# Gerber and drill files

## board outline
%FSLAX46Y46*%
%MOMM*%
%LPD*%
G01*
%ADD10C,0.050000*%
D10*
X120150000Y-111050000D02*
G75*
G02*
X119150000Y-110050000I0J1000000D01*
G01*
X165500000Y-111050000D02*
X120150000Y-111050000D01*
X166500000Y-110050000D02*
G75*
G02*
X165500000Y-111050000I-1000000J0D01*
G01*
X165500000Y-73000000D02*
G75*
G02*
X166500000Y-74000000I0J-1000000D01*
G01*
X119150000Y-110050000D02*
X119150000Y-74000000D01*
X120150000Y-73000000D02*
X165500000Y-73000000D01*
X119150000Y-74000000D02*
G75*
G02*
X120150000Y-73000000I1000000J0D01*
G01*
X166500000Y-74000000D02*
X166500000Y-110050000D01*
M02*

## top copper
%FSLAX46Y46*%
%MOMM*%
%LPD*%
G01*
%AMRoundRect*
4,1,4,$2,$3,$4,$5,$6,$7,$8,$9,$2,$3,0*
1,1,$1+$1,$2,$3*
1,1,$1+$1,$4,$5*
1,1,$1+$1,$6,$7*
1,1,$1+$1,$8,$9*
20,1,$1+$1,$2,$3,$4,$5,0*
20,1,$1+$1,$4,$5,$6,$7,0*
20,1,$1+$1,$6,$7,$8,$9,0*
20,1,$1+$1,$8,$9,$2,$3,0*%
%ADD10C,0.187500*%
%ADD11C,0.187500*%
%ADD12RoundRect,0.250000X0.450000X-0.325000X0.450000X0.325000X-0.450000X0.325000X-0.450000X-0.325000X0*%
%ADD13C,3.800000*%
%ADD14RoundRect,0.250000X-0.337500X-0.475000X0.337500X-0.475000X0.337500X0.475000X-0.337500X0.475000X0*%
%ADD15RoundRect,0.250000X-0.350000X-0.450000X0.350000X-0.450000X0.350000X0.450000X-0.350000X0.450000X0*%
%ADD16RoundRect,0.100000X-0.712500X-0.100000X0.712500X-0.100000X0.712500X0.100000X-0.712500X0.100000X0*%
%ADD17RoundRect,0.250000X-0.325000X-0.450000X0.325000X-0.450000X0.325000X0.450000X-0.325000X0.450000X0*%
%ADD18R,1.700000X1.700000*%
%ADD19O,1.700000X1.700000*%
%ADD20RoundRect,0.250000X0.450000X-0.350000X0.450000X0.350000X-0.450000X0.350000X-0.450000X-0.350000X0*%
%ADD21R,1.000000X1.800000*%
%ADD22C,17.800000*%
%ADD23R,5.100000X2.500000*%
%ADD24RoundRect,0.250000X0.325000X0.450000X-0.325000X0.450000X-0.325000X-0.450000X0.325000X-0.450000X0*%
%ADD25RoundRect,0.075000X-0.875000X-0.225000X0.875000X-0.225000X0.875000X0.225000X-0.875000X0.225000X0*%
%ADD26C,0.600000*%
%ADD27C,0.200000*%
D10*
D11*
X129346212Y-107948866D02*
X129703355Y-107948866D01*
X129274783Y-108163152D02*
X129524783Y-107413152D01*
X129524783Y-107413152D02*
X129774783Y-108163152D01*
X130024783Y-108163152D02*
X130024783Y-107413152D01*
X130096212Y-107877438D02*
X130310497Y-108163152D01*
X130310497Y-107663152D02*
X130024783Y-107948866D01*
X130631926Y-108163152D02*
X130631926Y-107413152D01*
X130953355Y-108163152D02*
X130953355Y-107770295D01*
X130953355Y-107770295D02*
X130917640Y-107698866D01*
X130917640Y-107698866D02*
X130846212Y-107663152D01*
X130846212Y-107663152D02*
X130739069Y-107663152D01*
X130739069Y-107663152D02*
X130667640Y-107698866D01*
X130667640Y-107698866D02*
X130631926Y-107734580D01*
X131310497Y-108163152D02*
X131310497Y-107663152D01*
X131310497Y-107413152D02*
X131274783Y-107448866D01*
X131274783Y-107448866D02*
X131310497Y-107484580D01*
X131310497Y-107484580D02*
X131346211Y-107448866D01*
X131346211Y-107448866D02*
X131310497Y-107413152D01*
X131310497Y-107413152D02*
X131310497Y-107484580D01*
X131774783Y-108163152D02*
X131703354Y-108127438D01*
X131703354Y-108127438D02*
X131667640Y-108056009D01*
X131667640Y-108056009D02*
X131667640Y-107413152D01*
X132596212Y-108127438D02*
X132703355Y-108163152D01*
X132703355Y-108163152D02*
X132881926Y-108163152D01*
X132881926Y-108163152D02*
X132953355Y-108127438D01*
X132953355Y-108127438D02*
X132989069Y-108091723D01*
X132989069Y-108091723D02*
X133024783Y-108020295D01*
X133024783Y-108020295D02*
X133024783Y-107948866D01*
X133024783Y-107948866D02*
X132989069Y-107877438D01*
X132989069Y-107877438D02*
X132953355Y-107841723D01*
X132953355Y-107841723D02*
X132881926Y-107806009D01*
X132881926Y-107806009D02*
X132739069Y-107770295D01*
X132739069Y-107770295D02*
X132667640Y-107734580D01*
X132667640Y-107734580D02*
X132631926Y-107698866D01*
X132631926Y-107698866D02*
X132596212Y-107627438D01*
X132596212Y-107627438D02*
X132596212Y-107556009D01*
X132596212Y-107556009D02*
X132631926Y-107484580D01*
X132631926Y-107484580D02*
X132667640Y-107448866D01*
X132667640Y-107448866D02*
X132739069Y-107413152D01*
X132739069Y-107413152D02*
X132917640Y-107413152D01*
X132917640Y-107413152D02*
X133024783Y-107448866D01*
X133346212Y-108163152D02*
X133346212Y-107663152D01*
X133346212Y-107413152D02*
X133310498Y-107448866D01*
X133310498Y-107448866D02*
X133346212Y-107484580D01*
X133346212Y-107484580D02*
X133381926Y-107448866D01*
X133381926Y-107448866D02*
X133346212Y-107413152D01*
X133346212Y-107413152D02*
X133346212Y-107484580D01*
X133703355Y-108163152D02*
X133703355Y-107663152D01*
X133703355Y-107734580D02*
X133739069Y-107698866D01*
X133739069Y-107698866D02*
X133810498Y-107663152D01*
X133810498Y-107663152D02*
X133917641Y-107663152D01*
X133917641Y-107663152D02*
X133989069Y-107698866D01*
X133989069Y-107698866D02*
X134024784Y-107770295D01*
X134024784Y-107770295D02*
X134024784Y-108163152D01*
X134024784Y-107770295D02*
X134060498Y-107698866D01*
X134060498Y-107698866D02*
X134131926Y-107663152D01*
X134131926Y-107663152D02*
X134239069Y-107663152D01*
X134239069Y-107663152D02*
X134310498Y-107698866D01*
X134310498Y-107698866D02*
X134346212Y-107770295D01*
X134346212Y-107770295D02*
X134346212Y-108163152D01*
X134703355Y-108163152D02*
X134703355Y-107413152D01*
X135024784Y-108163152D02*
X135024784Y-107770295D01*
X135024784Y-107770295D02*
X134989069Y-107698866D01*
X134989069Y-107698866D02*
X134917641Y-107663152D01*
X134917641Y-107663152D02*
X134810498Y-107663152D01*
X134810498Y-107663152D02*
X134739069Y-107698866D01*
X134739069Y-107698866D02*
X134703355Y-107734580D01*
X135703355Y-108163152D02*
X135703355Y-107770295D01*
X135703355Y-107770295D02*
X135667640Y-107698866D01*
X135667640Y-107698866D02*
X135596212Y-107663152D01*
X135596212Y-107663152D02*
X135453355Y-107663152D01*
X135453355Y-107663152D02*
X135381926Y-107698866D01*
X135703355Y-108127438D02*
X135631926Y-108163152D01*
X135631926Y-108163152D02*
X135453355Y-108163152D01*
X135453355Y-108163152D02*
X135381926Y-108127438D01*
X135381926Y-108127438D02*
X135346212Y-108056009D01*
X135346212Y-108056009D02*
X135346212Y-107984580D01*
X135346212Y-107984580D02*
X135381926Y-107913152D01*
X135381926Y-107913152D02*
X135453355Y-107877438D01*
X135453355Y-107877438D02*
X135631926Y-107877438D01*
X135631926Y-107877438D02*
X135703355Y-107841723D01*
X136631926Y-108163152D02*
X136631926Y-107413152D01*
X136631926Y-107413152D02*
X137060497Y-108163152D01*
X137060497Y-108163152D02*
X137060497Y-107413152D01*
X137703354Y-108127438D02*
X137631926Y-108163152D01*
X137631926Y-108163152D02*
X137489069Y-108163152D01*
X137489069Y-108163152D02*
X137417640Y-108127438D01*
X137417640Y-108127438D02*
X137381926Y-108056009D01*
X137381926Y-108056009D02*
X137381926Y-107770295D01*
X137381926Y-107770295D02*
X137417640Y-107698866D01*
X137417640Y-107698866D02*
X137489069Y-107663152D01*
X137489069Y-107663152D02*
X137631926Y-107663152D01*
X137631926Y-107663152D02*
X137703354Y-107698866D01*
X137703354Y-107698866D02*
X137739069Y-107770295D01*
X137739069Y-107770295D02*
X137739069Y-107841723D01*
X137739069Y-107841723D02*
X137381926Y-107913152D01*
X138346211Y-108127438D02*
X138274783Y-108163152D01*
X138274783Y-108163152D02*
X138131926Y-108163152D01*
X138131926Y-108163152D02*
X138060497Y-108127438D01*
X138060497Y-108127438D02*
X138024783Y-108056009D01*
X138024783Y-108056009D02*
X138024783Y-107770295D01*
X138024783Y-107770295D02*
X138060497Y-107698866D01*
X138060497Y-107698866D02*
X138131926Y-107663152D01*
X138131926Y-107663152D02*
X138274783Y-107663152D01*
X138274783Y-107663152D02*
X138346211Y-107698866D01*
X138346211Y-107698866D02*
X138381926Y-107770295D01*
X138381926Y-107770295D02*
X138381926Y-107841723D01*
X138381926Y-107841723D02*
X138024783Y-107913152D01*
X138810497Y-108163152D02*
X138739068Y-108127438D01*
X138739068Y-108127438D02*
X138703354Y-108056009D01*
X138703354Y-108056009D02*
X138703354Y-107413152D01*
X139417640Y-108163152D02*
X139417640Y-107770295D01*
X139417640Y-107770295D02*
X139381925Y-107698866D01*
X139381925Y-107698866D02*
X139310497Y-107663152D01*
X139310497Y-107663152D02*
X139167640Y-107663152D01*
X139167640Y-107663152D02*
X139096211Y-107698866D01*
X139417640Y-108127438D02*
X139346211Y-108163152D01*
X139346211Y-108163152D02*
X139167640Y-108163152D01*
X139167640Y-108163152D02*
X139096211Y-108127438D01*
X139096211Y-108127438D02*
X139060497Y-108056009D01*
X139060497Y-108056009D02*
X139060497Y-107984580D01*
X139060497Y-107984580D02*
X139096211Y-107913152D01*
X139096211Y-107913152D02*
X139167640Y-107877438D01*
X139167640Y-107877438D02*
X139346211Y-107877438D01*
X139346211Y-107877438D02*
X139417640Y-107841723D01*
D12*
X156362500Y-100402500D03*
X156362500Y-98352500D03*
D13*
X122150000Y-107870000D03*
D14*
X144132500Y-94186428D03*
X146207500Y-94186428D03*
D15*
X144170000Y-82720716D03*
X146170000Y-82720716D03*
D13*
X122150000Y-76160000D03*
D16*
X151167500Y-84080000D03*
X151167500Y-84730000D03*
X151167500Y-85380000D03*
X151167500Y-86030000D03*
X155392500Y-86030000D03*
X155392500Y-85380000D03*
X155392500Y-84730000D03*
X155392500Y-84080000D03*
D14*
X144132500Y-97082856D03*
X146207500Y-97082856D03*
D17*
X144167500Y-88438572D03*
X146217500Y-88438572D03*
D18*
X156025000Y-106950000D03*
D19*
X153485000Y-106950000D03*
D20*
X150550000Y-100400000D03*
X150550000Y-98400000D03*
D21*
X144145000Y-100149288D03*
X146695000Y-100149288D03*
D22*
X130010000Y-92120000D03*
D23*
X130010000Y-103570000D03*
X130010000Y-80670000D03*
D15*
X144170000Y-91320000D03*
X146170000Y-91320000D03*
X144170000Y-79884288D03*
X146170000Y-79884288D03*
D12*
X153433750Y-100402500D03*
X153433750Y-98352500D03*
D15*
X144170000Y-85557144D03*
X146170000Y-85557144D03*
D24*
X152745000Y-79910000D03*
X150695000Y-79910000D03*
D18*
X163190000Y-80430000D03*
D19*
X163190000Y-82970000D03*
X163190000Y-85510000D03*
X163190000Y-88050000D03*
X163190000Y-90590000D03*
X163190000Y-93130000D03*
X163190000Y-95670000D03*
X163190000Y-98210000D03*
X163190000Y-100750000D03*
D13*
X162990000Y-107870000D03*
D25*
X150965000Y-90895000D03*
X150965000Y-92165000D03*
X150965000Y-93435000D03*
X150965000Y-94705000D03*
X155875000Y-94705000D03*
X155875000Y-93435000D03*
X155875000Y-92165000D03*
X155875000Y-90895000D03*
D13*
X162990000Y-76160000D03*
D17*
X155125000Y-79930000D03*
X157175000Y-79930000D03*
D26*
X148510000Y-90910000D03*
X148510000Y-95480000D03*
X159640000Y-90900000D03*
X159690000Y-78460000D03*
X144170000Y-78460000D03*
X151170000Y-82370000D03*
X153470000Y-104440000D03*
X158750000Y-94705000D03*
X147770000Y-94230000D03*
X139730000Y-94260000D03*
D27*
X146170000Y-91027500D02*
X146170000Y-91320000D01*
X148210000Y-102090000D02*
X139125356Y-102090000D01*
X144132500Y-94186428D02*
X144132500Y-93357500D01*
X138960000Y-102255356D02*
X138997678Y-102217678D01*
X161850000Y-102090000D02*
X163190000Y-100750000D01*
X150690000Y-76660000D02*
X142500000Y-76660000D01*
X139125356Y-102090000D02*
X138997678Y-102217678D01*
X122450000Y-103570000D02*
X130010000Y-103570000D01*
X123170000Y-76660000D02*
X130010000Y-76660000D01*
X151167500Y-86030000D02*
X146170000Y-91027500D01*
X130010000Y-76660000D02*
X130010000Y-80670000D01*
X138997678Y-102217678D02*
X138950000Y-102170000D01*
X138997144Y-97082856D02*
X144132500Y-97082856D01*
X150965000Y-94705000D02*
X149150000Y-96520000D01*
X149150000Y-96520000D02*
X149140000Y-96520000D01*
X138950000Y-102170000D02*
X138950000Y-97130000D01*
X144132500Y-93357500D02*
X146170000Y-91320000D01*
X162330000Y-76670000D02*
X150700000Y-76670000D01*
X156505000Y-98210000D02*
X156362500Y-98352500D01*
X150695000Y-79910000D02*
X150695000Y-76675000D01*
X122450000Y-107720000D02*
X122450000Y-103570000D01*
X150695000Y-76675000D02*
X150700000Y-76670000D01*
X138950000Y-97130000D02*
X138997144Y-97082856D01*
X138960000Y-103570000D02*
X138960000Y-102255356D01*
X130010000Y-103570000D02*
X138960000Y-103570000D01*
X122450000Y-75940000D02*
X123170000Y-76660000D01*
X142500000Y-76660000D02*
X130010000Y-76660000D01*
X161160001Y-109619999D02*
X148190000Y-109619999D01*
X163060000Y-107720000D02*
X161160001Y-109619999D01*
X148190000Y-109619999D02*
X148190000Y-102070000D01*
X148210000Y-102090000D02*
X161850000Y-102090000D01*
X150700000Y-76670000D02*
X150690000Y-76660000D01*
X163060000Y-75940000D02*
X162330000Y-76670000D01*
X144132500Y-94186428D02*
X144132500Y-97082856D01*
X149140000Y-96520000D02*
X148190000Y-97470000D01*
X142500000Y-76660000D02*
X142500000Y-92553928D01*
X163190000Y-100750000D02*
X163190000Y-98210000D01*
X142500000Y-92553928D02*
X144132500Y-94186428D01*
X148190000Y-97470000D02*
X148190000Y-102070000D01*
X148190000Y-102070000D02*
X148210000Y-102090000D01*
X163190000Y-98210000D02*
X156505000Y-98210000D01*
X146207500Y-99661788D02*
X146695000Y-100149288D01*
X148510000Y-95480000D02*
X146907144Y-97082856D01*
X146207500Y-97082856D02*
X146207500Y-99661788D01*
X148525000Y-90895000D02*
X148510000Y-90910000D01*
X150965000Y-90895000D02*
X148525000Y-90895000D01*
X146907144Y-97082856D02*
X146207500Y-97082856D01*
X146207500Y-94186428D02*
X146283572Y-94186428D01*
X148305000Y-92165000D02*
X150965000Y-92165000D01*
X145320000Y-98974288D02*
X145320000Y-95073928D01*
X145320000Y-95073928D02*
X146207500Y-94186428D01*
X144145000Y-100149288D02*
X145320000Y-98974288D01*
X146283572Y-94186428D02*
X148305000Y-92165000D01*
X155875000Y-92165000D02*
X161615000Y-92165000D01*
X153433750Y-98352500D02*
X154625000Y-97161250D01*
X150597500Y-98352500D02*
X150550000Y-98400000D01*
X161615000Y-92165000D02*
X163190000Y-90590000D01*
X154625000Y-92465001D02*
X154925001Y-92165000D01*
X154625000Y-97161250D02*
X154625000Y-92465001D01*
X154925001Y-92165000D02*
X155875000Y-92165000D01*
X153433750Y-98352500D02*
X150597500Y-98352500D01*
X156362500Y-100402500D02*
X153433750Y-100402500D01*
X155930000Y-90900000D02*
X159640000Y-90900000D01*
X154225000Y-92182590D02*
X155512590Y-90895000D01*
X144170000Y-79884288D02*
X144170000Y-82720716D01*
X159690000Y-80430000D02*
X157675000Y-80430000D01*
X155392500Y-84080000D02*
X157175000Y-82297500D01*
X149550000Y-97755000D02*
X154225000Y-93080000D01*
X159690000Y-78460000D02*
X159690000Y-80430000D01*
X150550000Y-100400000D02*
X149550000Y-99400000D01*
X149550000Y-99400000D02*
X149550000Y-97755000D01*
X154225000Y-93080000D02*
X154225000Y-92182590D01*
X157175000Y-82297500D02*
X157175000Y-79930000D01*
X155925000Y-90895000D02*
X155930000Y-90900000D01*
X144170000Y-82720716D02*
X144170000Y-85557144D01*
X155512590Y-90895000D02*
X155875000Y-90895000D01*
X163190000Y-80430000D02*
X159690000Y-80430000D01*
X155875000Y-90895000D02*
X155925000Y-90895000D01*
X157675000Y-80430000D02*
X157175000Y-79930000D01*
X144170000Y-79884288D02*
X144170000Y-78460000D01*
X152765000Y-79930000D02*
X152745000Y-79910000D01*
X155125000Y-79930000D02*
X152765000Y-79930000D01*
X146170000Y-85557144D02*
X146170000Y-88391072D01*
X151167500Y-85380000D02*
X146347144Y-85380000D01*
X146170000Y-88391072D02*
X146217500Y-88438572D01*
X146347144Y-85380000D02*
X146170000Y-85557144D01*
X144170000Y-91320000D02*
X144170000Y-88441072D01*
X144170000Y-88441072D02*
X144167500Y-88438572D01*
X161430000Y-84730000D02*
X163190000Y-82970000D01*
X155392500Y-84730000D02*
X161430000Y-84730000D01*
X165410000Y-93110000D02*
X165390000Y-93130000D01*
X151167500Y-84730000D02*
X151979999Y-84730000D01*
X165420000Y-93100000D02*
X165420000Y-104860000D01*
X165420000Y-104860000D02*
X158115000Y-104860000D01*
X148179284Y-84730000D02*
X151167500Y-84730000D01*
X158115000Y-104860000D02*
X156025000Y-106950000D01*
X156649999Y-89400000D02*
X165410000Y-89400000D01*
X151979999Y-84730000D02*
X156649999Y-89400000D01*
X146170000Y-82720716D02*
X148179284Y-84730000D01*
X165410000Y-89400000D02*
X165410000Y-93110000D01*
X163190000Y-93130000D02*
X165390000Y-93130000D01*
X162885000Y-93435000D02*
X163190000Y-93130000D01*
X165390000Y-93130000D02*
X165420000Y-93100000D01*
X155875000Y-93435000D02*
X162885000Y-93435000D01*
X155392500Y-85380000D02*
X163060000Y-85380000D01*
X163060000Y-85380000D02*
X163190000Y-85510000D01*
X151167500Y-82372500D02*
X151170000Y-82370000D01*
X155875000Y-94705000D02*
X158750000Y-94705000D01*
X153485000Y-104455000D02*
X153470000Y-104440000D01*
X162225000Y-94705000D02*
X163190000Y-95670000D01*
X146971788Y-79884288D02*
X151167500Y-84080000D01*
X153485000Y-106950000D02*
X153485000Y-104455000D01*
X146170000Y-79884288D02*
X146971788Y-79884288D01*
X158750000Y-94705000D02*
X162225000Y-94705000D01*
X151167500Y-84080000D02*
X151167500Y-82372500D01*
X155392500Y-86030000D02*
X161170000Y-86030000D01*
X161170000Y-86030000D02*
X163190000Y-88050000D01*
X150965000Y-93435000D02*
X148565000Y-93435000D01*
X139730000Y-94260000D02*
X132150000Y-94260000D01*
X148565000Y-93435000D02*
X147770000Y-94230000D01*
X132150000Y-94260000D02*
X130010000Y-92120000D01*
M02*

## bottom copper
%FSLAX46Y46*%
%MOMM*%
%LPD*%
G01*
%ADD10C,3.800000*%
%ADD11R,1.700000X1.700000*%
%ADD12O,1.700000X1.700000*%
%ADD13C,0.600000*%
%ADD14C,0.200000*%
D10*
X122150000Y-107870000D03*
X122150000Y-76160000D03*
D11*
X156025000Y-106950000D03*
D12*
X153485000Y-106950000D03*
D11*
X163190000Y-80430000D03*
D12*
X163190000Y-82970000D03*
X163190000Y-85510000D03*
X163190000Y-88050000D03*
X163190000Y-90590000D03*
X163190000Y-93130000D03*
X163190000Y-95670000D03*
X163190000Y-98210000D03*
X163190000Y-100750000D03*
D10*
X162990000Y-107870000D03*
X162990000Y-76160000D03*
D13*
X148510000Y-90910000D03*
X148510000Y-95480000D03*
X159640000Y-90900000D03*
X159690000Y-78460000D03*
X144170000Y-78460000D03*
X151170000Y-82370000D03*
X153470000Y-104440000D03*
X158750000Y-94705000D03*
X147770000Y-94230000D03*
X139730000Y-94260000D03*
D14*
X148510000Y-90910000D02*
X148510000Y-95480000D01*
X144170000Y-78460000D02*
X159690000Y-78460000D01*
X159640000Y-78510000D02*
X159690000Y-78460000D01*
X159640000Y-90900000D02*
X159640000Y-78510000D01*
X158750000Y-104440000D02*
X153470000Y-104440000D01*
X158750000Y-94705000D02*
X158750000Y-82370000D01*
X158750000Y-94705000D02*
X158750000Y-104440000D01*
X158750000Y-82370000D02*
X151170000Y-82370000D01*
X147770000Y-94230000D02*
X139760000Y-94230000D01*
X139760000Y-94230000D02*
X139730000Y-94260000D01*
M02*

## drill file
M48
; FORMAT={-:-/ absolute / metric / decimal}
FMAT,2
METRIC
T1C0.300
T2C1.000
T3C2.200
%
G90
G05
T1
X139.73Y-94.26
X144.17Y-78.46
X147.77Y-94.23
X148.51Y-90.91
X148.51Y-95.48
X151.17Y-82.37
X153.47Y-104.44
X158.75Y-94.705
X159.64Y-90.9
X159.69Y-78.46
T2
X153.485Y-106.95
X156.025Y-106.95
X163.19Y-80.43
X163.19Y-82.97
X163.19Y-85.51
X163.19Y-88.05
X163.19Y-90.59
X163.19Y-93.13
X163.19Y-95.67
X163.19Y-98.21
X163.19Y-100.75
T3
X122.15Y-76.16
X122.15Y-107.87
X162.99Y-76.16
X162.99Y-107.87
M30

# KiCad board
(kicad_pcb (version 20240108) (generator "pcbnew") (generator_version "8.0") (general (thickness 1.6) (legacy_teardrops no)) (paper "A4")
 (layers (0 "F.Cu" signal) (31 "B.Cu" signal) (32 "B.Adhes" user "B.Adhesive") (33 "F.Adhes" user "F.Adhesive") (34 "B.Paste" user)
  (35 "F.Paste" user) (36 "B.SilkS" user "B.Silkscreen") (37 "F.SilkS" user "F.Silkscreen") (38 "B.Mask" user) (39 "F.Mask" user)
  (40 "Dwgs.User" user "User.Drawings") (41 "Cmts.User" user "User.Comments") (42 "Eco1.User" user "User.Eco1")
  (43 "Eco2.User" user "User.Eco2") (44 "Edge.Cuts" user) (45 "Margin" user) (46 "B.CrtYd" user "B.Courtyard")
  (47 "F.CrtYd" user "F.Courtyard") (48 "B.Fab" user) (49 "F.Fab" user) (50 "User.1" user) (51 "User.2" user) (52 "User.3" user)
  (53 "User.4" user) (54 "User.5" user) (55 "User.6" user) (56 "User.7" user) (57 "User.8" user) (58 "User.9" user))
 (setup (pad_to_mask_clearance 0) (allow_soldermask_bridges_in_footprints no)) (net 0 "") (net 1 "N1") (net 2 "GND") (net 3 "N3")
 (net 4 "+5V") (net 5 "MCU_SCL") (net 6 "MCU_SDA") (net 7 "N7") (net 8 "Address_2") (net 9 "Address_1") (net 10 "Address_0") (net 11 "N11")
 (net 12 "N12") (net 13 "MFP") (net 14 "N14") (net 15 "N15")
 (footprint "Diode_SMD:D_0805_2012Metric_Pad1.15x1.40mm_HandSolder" (layer "F.Cu") (at 156.3625 99.3775 90)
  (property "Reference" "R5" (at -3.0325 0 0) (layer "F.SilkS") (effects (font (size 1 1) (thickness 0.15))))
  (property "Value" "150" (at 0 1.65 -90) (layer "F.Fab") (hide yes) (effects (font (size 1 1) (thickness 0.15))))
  (pad "1" smd roundrect (at -1.025 0 90) (size 1.15 1.4) (layers "F.Cu" "F.Paste" "F.Mask") (roundrect_rratio 0.217391) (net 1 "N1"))
  (pad "2" smd roundrect (at 1.025 0 90) (size 1.15 1.4) (layers "F.Cu" "F.Paste" "F.Mask") (roundrect_rratio 0.217391) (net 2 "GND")))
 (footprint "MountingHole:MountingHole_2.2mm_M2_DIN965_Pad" (layer "F.Cu") (at 122.15 107.87)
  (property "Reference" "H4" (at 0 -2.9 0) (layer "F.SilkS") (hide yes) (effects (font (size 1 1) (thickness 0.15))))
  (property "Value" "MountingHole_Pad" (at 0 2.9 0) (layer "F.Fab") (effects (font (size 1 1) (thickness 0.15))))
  (pad "1" thru_hole circle (at 0 0) (size 3.8 3.8) (drill 2.2) (layers "*.Cu" "*.Mask") (remove_unused_layers no) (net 2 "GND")))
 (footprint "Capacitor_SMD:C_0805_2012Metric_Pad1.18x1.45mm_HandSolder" (layer "F.Cu") (at 145.17 94.186428)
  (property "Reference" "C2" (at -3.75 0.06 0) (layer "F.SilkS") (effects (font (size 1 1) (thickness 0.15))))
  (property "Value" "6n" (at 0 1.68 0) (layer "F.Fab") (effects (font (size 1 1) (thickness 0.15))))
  (pad "1" smd roundrect (at -1.0375 0) (size 1.175 1.45) (layers "F.Cu" "F.Paste" "F.Mask") (roundrect_rratio 0.212766) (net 2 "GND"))
  (pad "2" smd roundrect (at 1.0375 0) (size 1.175 1.45) (layers "F.Cu" "F.Paste" "F.Mask") (roundrect_rratio 0.212766) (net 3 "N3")))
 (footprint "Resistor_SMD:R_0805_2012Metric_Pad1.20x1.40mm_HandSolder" (layer "F.Cu") (at 145.17 82.720716)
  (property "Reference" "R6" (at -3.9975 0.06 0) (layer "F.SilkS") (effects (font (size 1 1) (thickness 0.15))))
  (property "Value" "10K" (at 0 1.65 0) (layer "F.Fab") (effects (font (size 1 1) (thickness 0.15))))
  (pad "1" smd roundrect (at -1 0) (size 1.2 1.4) (layers "F.Cu" "F.Paste" "F.Mask") (roundrect_rratio 0.208333) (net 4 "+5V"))
  (pad "2" smd roundrect (at 1 0) (size 1.2 1.4) (layers "F.Cu" "F.Paste" "F.Mask") (roundrect_rratio 0.208333) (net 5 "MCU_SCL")))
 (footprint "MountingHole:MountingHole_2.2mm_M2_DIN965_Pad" (layer "F.Cu") (at 122.15 76.16)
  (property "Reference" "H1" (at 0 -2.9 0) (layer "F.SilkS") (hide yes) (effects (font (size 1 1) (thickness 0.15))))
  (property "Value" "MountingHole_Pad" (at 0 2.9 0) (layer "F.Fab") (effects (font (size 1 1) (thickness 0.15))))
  (pad "1" thru_hole circle (at 0 0) (size 3.8 3.8) (drill 2.2) (layers "*.Cu" "*.Mask") (remove_unused_layers no) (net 2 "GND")))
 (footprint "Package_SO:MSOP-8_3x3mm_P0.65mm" (layer "F.Cu") (at 153.28 85.055)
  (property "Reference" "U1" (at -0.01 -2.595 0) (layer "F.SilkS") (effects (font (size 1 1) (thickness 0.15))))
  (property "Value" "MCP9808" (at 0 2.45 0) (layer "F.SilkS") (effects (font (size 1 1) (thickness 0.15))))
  (pad "1" smd roundrect (at -2.1125 -0.975) (size 1.625 0.4) (layers "F.Cu" "F.Paste" "F.Mask") (roundrect_rratio 0.25) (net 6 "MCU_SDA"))
  (pad "2" smd roundrect (at -2.1125 -0.325) (size 1.625 0.4) (layers "F.Cu" "F.Paste" "F.Mask") (roundrect_rratio 0.25) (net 5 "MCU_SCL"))
  (pad "3" smd roundrect (at -2.1125 0.325) (size 1.625 0.4) (layers "F.Cu" "F.Paste" "F.Mask") (roundrect_rratio 0.25) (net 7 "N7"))
  (pad "4" smd roundrect (at -2.1125 0.975) (size 1.625 0.4) (layers "F.Cu" "F.Paste" "F.Mask") (roundrect_rratio 0.25) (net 2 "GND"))
  (pad "5" smd roundrect (at 2.1125 0.975) (size 1.625 0.4) (layers "F.Cu" "F.Paste" "F.Mask") (roundrect_rratio 0.25) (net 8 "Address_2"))
  (pad "6" smd roundrect (at 2.1125 0.325) (size 1.625 0.4) (layers "F.Cu" "F.Paste" "F.Mask") (roundrect_rratio 0.25) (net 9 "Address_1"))
  (pad "7" smd roundrect (at 2.1125 -0.325) (size 1.625 0.4) (layers "F.Cu" "F.Paste" "F.Mask") (roundrect_rratio 0.25) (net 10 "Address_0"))
  (pad "8" smd roundrect (at 2.1125 -0.975) (size 1.625 0.4) (layers "F.Cu" "F.Paste" "F.Mask") (roundrect_rratio 0.25) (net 4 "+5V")))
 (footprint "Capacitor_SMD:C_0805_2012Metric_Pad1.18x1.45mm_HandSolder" (layer "F.Cu") (at 145.17 97.082856)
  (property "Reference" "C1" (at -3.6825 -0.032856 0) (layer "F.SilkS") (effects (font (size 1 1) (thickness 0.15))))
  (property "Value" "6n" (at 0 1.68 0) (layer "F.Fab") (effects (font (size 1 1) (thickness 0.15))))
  (pad "1" smd roundrect (at -1.0375 0) (size 1.175 1.45) (layers "F.Cu" "F.Paste" "F.Mask") (roundrect_rratio 0.212766) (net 2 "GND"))
  (pad "2" smd roundrect (at 1.0375 0) (size 1.175 1.45) (layers "F.Cu" "F.Paste" "F.Mask") (roundrect_rratio 0.212766) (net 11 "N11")))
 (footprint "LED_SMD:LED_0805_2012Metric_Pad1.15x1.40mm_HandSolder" (layer "F.Cu") (at 145.1925 88.438572)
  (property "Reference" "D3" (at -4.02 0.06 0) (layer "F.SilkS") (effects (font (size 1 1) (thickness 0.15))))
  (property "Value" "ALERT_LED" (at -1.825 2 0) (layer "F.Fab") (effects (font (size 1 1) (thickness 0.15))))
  (pad "1" smd roundrect (at -1.025 0) (size 1.15 1.4) (layers "F.Cu" "F.Paste" "F.Mask") (roundrect_rratio 0.217391) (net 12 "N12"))
  (pad "2" smd roundrect (at 1.025 0) (size 1.15 1.4) (layers "F.Cu" "F.Paste" "F.Mask") (roundrect_rratio 0.217391) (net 7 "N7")))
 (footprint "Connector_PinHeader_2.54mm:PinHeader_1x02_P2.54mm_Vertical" (layer "F.Cu") (at 156.025 106.95 -90)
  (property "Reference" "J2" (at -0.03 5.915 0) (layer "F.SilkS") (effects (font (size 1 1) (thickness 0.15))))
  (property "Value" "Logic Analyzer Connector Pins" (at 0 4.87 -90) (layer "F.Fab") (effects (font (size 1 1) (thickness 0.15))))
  (pad "1" thru_hole rect (at 0 0 270) (size 1.7 1.7) (drill 1) (layers "*.Cu" "*.Mask") (remove_unused_layers no) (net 5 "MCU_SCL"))
  (pad "2" thru_hole oval (at 0 2.54 270) (size 1.7 1.7) (drill 1) (layers "*.Cu" "*.Mask") (remove_unused_layers no) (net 6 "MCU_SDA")))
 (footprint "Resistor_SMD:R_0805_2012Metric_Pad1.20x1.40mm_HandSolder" (layer "F.Cu") (at 150.55 99.4 90)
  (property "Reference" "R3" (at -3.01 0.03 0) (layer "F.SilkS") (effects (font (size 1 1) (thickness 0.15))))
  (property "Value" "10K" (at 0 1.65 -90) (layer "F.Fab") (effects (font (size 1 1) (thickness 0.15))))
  (pad "1" smd roundrect (at -1 0 90) (size 1.2 1.4) (layers "F.Cu" "F.Paste" "F.Mask") (roundrect_rratio 0.208333) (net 4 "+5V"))
  (pad "2" smd roundrect (at 1 0 90) (size 1.2 1.4) (layers "F.Cu" "F.Paste" "F.Mask") (roundrect_rratio 0.208333) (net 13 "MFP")))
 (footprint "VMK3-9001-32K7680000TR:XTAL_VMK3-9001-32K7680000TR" (layer "F.Cu") (at 145.42 100.149288)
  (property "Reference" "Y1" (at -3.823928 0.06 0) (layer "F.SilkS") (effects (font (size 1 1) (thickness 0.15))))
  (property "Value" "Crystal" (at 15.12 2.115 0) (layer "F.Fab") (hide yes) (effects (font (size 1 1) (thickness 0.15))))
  (pad "1" smd rect (at -1.275 0) (size 1 1.8) (layers "F.Cu" "F.Paste" "F.Mask") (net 3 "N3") (solder_mask_margin 0.102))
  (pad "2" smd rect (at 1.275 0) (size 1 1.8) (layers "F.Cu" "F.Paste" "F.Mask") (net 11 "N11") (solder_mask_margin 0.102)))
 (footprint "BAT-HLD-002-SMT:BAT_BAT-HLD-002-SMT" (layer "F.Cu") (at 130.01 92.12 90)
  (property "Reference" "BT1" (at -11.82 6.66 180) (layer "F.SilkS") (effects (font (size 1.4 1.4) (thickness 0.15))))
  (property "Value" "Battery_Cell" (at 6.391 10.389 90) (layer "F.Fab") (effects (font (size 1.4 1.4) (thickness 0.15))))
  (pad "N" smd circle (at 0 0 90) (size 17.8 17.8) (layers "F.Cu" "F.Mask") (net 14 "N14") (solder_mask_margin 0.102))
  (pad "P1" smd rect (at -11.45 0 90) (size 2.5 5.1) (layers "F.Cu" "F.Paste" "F.Mask") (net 2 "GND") (solder_mask_margin 0.102))
  (pad "P2" smd rect (at 11.45 0 90) (size 2.5 5.1) (layers "F.Cu" "F.Paste" "F.Mask") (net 2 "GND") (solder_mask_margin 0.102)))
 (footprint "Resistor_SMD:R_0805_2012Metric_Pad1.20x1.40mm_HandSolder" (layer "F.Cu") (at 145.17 91.32)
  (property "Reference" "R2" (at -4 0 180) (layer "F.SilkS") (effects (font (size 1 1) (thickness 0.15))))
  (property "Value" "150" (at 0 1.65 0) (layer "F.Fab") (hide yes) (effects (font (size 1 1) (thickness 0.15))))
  (pad "1" smd roundrect (at -1 0) (size 1.2 1.4) (layers "F.Cu" "F.Paste" "F.Mask") (roundrect_rratio 0.208333) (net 12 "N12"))
  (pad "2" smd roundrect (at 1 0) (size 1.2 1.4) (layers "F.Cu" "F.Paste" "F.Mask") (roundrect_rratio 0.208333) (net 2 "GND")))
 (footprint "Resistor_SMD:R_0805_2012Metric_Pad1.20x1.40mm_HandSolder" (layer "F.Cu") (at 145.17 79.884288)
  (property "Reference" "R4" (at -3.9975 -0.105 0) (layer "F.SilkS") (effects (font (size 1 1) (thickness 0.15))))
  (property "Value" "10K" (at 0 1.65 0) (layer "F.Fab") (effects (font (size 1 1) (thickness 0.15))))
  (pad "1" smd roundrect (at -1 0) (size 1.2 1.4) (layers "F.Cu" "F.Paste" "F.Mask") (roundrect_rratio 0.208333) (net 4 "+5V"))
  (pad "2" smd roundrect (at 1 0) (size 1.2 1.4) (layers "F.Cu" "F.Paste" "F.Mask") (roundrect_rratio 0.208333) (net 6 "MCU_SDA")))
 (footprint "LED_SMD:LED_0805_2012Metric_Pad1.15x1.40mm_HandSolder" (layer "F.Cu") (at 153.43375 99.3775 90)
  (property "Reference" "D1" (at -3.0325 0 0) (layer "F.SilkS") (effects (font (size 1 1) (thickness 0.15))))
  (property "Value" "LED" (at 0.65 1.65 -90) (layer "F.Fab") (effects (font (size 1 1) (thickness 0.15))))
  (pad "1" smd roundrect (at -1.025 0 90) (size 1.15 1.4) (layers "F.Cu" "F.Paste" "F.Mask") (roundrect_rratio 0.217391) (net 1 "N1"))
  (pad "2" smd roundrect (at 1.025 0 90) (size 1.15 1.4) (layers "F.Cu" "F.Paste" "F.Mask") (roundrect_rratio 0.217391) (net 13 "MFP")))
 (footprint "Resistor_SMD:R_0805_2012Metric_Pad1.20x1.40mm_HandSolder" (layer "F.Cu") (at 145.17 85.557144)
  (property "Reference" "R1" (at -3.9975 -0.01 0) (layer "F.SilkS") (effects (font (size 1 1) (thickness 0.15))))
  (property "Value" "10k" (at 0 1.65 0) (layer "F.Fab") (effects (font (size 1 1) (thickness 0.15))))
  (pad "1" smd roundrect (at -1 0) (size 1.2 1.4) (layers "F.Cu" "F.Paste" "F.Mask") (roundrect_rratio 0.208333) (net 4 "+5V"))
  (pad "2" smd roundrect (at 1 0) (size 1.2 1.4) (layers "F.Cu" "F.Paste" "F.Mask") (roundrect_rratio 0.208333) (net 7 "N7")))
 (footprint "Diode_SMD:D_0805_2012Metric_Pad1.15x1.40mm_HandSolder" (layer "F.Cu") (at 151.72 79.91 180)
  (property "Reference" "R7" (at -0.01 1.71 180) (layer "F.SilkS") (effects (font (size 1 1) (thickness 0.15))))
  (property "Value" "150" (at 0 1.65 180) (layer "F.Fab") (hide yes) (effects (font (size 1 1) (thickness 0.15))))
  (pad "1" smd roundrect (at -1.025 0 180) (size 1.15 1.4) (layers "F.Cu" "F.Paste" "F.Mask") (roundrect_rratio 0.217391) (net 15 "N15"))
  (pad "2" smd roundrect (at 1.025 0 180) (size 1.15 1.4) (layers "F.Cu" "F.Paste" "F.Mask") (roundrect_rratio 0.217391) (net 2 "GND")))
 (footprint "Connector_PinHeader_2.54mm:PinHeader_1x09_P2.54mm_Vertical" (layer "F.Cu") (at 163.19 80.43)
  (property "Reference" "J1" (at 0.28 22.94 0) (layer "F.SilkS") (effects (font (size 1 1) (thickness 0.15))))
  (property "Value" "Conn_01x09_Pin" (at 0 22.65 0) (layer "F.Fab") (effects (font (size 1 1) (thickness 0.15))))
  (pad "1" thru_hole rect (at 0 0) (size 1.7 1.7) (drill 1) (layers "*.Cu" "*.Mask") (remove_unused_layers no) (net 4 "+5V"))
  (pad "2" thru_hole oval (at 0 2.54) (size 1.7 1.7) (drill 1) (layers "*.Cu" "*.Mask") (remove_unused_layers no) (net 10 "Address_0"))
  (pad "3" thru_hole oval (at 0 5.08) (size 1.7 1.7) (drill 1) (layers "*.Cu" "*.Mask") (remove_unused_layers no) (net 9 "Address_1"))
  (pad "4" thru_hole oval (at 0 7.62) (size 1.7 1.7) (drill 1) (layers "*.Cu" "*.Mask") (remove_unused_layers no) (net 8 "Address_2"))
  (pad "5" thru_hole oval (at 0 10.16) (size 1.7 1.7) (drill 1) (layers "*.Cu" "*.Mask") (remove_unused_layers no) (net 13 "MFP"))
  (pad "6" thru_hole oval (at 0 12.7) (size 1.7 1.7) (drill 1) (layers "*.Cu" "*.Mask") (remove_unused_layers no) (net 5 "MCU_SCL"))
  (pad "7" thru_hole oval (at 0 15.24) (size 1.7 1.7) (drill 1) (layers "*.Cu" "*.Mask") (remove_unused_layers no) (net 6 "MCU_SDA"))
  (pad "8" thru_hole oval (at 0 17.78) (size 1.7 1.7) (drill 1) (layers "*.Cu" "*.Mask") (remove_unused_layers no) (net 2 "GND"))
  (pad "9" thru_hole oval (at 0 20.32) (size 1.7 1.7) (drill 1) (layers "*.Cu" "*.Mask") (remove_unused_layers no) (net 2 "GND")))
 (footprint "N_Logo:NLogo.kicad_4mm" (layer "F.Cu") (at 127.06 107.719644)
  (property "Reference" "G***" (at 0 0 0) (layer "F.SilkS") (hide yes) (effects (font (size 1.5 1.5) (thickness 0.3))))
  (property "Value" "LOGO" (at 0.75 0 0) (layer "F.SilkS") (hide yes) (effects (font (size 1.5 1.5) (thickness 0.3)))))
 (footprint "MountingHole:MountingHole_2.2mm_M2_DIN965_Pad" (layer "F.Cu") (at 162.99 107.87)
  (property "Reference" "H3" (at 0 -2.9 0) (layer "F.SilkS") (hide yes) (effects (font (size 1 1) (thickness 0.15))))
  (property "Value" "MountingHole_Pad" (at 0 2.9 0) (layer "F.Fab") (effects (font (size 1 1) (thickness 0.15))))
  (pad "1" thru_hole circle (at 0 0) (size 3.8 3.8) (drill 2.2) (layers "*.Cu" "*.Mask") (remove_unused_layers no) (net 2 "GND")))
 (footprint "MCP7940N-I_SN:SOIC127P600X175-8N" (layer "F.Cu") (at 153.42 92.8)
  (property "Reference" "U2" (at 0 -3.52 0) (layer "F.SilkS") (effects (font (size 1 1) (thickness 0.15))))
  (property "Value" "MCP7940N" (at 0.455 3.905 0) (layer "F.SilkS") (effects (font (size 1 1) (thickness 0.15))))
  (pad "1" smd roundrect (at -2.455 -1.905) (size 1.9 0.6) (layers "F.Cu" "F.Paste" "F.Mask") (roundrect_rratio 0.125) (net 11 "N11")
   (solder_mask_margin 0.102))
  (pad "2" smd roundrect (at -2.455 -0.635) (size 1.9 0.6) (layers "F.Cu" "F.Paste" "F.Mask") (roundrect_rratio 0.125) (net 3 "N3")
   (solder_mask_margin 0.102))
  (pad "3" smd roundrect (at -2.455 0.635) (size 1.9 0.6) (layers "F.Cu" "F.Paste" "F.Mask") (roundrect_rratio 0.125) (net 14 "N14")
   (solder_mask_margin 0.102))
  (pad "4" smd roundrect (at -2.455 1.905) (size 1.9 0.6) (layers "F.Cu" "F.Paste" "F.Mask") (roundrect_rratio 0.125) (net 2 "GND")
   (solder_mask_margin 0.102))
  (pad "5" smd roundrect (at 2.455 1.905) (size 1.9 0.6) (layers "F.Cu" "F.Paste" "F.Mask") (roundrect_rratio 0.125) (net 6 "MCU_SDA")
   (solder_mask_margin 0.102))
  (pad "6" smd roundrect (at 2.455 0.635) (size 1.9 0.6) (layers "F.Cu" "F.Paste" "F.Mask") (roundrect_rratio 0.125) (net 5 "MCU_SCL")
   (solder_mask_margin 0.102))
  (pad "7" smd roundrect (at 2.455 -0.635) (size 1.9 0.6) (layers "F.Cu" "F.Paste" "F.Mask") (roundrect_rratio 0.125) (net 13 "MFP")
   (solder_mask_margin 0.102))
  (pad "8" smd roundrect (at 2.455 -1.905) (size 1.9 0.6) (layers "F.Cu" "F.Paste" "F.Mask") (roundrect_rratio 0.125) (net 4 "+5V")
   (solder_mask_margin 0.102)))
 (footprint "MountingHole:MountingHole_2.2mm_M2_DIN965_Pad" (layer "F.Cu") (at 162.99 76.16)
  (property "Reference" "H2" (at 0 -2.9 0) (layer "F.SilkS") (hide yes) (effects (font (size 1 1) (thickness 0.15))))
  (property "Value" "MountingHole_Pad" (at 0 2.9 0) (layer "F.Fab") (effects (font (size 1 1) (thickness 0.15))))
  (pad "1" thru_hole circle (at 0 0) (size 3.8 3.8) (drill 2.2) (layers "*.Cu" "*.Mask") (remove_unused_layers no) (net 2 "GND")))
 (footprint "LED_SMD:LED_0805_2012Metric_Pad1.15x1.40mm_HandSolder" (layer "F.Cu") (at 156.15 79.93)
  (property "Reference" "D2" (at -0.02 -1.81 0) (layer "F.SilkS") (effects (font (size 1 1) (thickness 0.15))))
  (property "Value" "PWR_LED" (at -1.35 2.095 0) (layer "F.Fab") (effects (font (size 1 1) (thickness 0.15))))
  (pad "1" smd roundrect (at -1.025 0) (size 1.15 1.4) (layers "F.Cu" "F.Paste" "F.Mask") (roundrect_rratio 0.217391) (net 15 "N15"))
  (pad "2" smd roundrect (at 1.025 0) (size 1.15 1.4) (layers "F.Cu" "F.Paste" "F.Mask") (roundrect_rratio 0.217391) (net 4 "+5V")))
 (gr_arc (start 120.15 111.05) (mid 119.442893 110.757107) (end 119.15 110.05) (stroke (width 0.05) (type default)) (layer "Edge.Cuts"))
 (gr_line (start 165.5 111.05) (end 120.15 111.05) (stroke (width 0.05) (type default)) (layer "Edge.Cuts"))
 (gr_arc (start 166.5 110.05) (mid 166.207107 110.757107) (end 165.5 111.05) (stroke (width 0.05) (type default)) (layer "Edge.Cuts"))
 (gr_arc (start 165.5 73) (mid 166.207107 73.292893) (end 166.5 74) (stroke (width 0.05) (type default)) (layer "Edge.Cuts"))
 (gr_line (start 119.15 110.05) (end 119.15 74) (stroke (width 0.05) (type default)) (layer "Edge.Cuts"))
 (gr_line (start 120.15 73) (end 165.5 73) (stroke (width 0.05) (type default)) (layer "Edge.Cuts"))
 (gr_arc (start 119.15 74) (mid 119.442893 73.292893) (end 120.15 73) (stroke (width 0.05) (type default)) (layer "Edge.Cuts"))
 (gr_line (start 166.5 74) (end 166.5 110.05) (stroke (width 0.05) (type default)) (layer "Edge.Cuts"))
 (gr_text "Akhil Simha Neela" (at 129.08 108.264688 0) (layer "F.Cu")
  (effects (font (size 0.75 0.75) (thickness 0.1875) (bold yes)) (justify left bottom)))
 (segment (start 146.17 91.0275) (end 146.17 91.32) (width 0.2) (layer "F.Cu") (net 2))
 (segment (start 148.21 102.09) (end 139.125356 102.09) (width 0.2) (layer "F.Cu") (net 2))
 (segment (start 144.1325 94.186428) (end 144.1325 93.3575) (width 0.2) (layer "F.Cu") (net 2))
 (segment (start 138.96 102.255356) (end 138.997678 102.217678) (width 0.2) (layer "F.Cu") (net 2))
 (segment (start 161.85 102.09) (end 163.19 100.75) (width 0.2) (layer "F.Cu") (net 2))
 (segment (start 150.69 76.66) (end 142.5 76.66) (width 0.2) (layer "F.Cu") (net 2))
 (segment (start 139.125356 102.09) (end 138.997678 102.217678) (width 0.2) (layer "F.Cu") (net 2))
 (segment (start 122.45 103.57) (end 130.01 103.57) (width 0.2) (layer "F.Cu") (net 2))
 (segment (start 123.17 76.66) (end 130.01 76.66) (width 0.2) (layer "F.Cu") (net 2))
 (segment (start 151.1675 86.03) (end 146.17 91.0275) (width 0.2) (layer "F.Cu") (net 2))
 (segment (start 130.01 76.66) (end 130.01 80.67) (width 0.2) (layer "F.Cu") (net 2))
 (segment (start 138.997678 102.217678) (end 138.95 102.17) (width 0.2) (layer "F.Cu") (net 2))
 (segment (start 138.997144 97.082856) (end 144.1325 97.082856) (width 0.2) (layer "F.Cu") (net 2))
 (segment (start 150.965 94.705) (end 149.15 96.52) (width 0.2) (layer "F.Cu") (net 2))
 (segment (start 149.15 96.52) (end 149.14 96.52) (width 0.2) (layer "F.Cu") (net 2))
 (segment (start 138.95 102.17) (end 138.95 97.13) (width 0.2) (layer "F.Cu") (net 2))
 (segment (start 144.1325 93.3575) (end 146.17 91.32) (width 0.2) (layer "F.Cu") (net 2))
 (segment (start 162.33 76.67) (end 150.7 76.67) (width 0.2) (layer "F.Cu") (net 2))
 (segment (start 156.505 98.21) (end 156.3625 98.3525) (width 0.2) (layer "F.Cu") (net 2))
 (segment (start 150.695 79.91) (end 150.695 76.675) (width 0.2) (layer "F.Cu") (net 2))
 (segment (start 122.45 107.72) (end 122.45 103.57) (width 0.2) (layer "F.Cu") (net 2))
 (segment (start 150.695 76.675) (end 150.7 76.67) (width 0.2) (layer "F.Cu") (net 2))
 (segment (start 138.95 97.13) (end 138.997144 97.082856) (width 0.2) (layer "F.Cu") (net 2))
 (segment (start 138.96 103.57) (end 138.96 102.255356) (width 0.2) (layer "F.Cu") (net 2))
 (segment (start 130.01 103.57) (end 138.96 103.57) (width 0.2) (layer "F.Cu") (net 2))
 (segment (start 122.45 75.94) (end 123.17 76.66) (width 0.2) (layer "F.Cu") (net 2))
 (segment (start 142.5 76.66) (end 130.01 76.66) (width 0.2) (layer "F.Cu") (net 2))
 (segment (start 161.160001 109.619999) (end 148.19 109.619999) (width 0.2) (layer "F.Cu") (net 2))
 (segment (start 163.06 107.72) (end 161.160001 109.619999) (width 0.2) (layer "F.Cu") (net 2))
 (segment (start 148.19 109.619999) (end 148.19 102.07) (width 0.2) (layer "F.Cu") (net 2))
 (segment (start 148.21 102.09) (end 161.85 102.09) (width 0.2) (layer "F.Cu") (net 2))
 (segment (start 150.7 76.67) (end 150.69 76.66) (width 0.2) (layer "F.Cu") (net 2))
 (segment (start 163.06 75.94) (end 162.33 76.67) (width 0.2) (layer "F.Cu") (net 2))
 (segment (start 144.1325 94.186428) (end 144.1325 97.082856) (width 0.2) (layer "F.Cu") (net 2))
 (segment (start 149.14 96.52) (end 148.19 97.47) (width 0.2) (layer "F.Cu") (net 2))
 (segment (start 142.5 76.66) (end 142.5 92.553928) (width 0.2) (layer "F.Cu") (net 2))
 (segment (start 163.19 100.75) (end 163.19 98.21) (width 0.2) (layer "F.Cu") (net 2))
 (segment (start 142.5 92.553928) (end 144.1325 94.186428) (width 0.2) (layer "F.Cu") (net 2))
 (segment (start 148.19 97.47) (end 148.19 102.07) (width 0.2) (layer "F.Cu") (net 2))
 (segment (start 148.19 102.07) (end 148.21 102.09) (width 0.2) (layer "F.Cu") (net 2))
 (segment (start 163.19 98.21) (end 156.505 98.21) (width 0.2) (layer "F.Cu") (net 2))
 (segment (start 146.2075 99.661788) (end 146.695 100.149288) (width 0.2) (layer "F.Cu") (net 11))
 (segment (start 148.51 95.48) (end 146.907144 97.082856) (width 0.2) (layer "F.Cu") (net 11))
 (segment (start 146.2075 97.082856) (end 146.2075 99.661788) (width 0.2) (layer "F.Cu") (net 11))
 (segment (start 148.525 90.895) (end 148.51 90.91) (width 0.2) (layer "F.Cu") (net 11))
 (segment (start 150.965 90.895) (end 148.525 90.895) (width 0.2) (layer "F.Cu") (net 11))
 (segment (start 146.907144 97.082856) (end 146.2075 97.082856) (width 0.2) (layer "F.Cu") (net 11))
 (via (at 148.51 90.91) (size 0.6) (drill 0.3) (layers "F.Cu" "B.Cu") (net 11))
 (via (at 148.51 95.48) (size 0.6) (drill 0.3) (layers "F.Cu" "B.Cu") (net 11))
 (segment (start 148.51 90.91) (end 148.51 95.48) (width 0.2) (layer "B.Cu") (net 11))
 (segment (start 146.2075 94.186428) (end 146.283572 94.186428) (width 0.2) (layer "F.Cu") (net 3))
 (segment (start 148.305 92.165) (end 150.965 92.165) (width 0.2) (layer "F.Cu") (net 3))
 (segment (start 145.32 98.974288) (end 145.32 95.073928) (width 0.2) (layer "F.Cu") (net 3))
 (segment (start 145.32 95.073928) (end 146.2075 94.186428) (width 0.2) (layer "F.Cu") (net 3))
 (segment (start 144.145 100.149288) (end 145.32 98.974288) (width 0.2) (layer "F.Cu") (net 3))
 (segment (start 146.283572 94.186428) (end 148.305 92.165) (width 0.2) (layer "F.Cu") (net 3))
 (segment (start 155.875 92.165) (end 161.615 92.165) (width 0.2) (layer "F.Cu") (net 13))
 (segment (start 153.43375 98.3525) (end 154.625 97.16125) (width 0.2) (layer "F.Cu") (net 13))
 (segment (start 150.5975 98.3525) (end 150.55 98.4) (width 0.2) (layer "F.Cu") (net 13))
 (segment (start 161.615 92.165) (end 163.19 90.59) (width 0.2) (layer "F.Cu") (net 13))
 (segment (start 154.625 92.465001) (end 154.925001 92.165) (width 0.2) (layer "F.Cu") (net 13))
 (segment (start 154.625 97.16125) (end 154.625 92.465001) (width 0.2) (layer "F.Cu") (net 13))
 (segment (start 154.925001 92.165) (end 155.875 92.165) (width 0.2) (layer "F.Cu") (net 13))
 (segment (start 153.43375 98.3525) (end 150.5975 98.3525) (width 0.2) (layer "F.Cu") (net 13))
 (segment (start 156.3625 100.4025) (end 153.43375 100.4025) (width 0.2) (layer "F.Cu") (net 1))
 (segment (start 155.93 90.9) (end 159.64 90.9) (width 0.2) (layer "F.Cu") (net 4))
 (segment (start 154.225 92.18259) (end 155.51259 90.895) (width 0.2) (layer "F.Cu") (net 4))
 (segment (start 144.17 79.884288) (end 144.17 82.720716) (width 0.2) (layer "F.Cu") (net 4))
 (segment (start 159.69 80.43) (end 157.675 80.43) (width 0.2) (layer "F.Cu") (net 4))
 (segment (start 155.3925 84.08) (end 157.175 82.2975) (width 0.2) (layer "F.Cu") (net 4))
 (segment (start 149.55 97.755) (end 154.225 93.08) (width 0.2) (layer "F.Cu") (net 4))
 (segment (start 159.69 78.46) (end 159.69 80.43) (width 0.2) (layer "F.Cu") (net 4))
 (segment (start 150.55 100.4) (end 149.55 99.4) (width 0.2) (layer "F.Cu") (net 4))
 (segment (start 149.55 99.4) (end 149.55 97.755) (width 0.2) (layer "F.Cu") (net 4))
 (segment (start 154.225 93.08) (end 154.225 92.18259) (width 0.2) (layer "F.Cu") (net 4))
 (segment (start 157.175 82.2975) (end 157.175 79.93) (width 0.2) (layer "F.Cu") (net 4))
 (segment (start 155.925 90.895) (end 155.93 90.9) (width 0.2) (layer "F.Cu") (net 4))
 (segment (start 144.17 82.720716) (end 144.17 85.557144) (width 0.2) (layer "F.Cu") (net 4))
 (segment (start 155.51259 90.895) (end 155.875 90.895) (width 0.2) (layer "F.Cu") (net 4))
 (segment (start 163.19 80.43) (end 159.69 80.43) (width 0.2) (layer "F.Cu") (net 4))
 (segment (start 155.875 90.895) (end 155.925 90.895) (width 0.2) (layer "F.Cu") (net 4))
 (segment (start 157.675 80.43) (end 157.175 79.93) (width 0.2) (layer "F.Cu") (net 4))
 (segment (start 144.17 79.884288) (end 144.17 78.46) (width 0.2) (layer "F.Cu") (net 4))
 (via (at 159.64 90.9) (size 0.6) (drill 0.3) (layers "F.Cu" "B.Cu") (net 4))
 (via (at 159.69 78.46) (size 0.6) (drill 0.3) (layers "F.Cu" "B.Cu") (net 4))
 (via (at 144.17 78.46) (size 0.6) (drill 0.3) (layers "F.Cu" "B.Cu") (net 4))
 (segment (start 144.17 78.46) (end 159.69 78.46) (width 0.2) (layer "B.Cu") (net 4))
 (segment (start 159.64 78.51) (end 159.69 78.46) (width 0.2) (layer "B.Cu") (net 4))
 (segment (start 159.64 90.9) (end 159.64 78.51) (width 0.2) (layer "B.Cu") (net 4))
 (segment (start 152.765 79.93) (end 152.745 79.91) (width 0.2) (layer "F.Cu") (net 15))
 (segment (start 155.125 79.93) (end 152.765 79.93) (width 0.2) (layer "F.Cu") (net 15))
 (segment (start 146.17 85.557144) (end 146.17 88.391072) (width 0.2) (layer "F.Cu") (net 7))
 (segment (start 151.1675 85.38) (end 146.347144 85.38) (width 0.2) (layer "F.Cu") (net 7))
 (segment (start 146.17 88.391072) (end 146.2175 88.438572) (width 0.2) (layer "F.Cu") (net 7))
 (segment (start 146.347144 85.38) (end 146.17 85.557144) (width 0.2) (layer "F.Cu") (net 7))
 (segment (start 144.17 91.32) (end 144.17 88.441072) (width 0.2) (layer "F.Cu") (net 12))
 (segment (start 144.17 88.441072) (end 144.1675 88.438572) (width 0.2) (layer "F.Cu") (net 12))
 (segment (start 161.43 84.73) (end 163.19 82.97) (width 0.2) (layer "F.Cu") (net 10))
 (segment (start 155.3925 84.73) (end 161.43 84.73) (width 0.2) (layer "F.Cu") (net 10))
 (segment (start 165.41 93.11) (end 165.39 93.13) (width 0.2) (layer "F.Cu") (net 5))
 (segment (start 151.1675 84.73) (end 151.979999 84.73) (width 0.2) (layer "F.Cu") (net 5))
 (segment (start 165.42 93.1) (end 165.42 104.86) (width 0.2) (layer "F.Cu") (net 5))
 (segment (start 165.42 104.86) (end 158.115 104.86) (width 0.2) (layer "F.Cu") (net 5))
 (segment (start 148.179284 84.73) (end 151.1675 84.73) (width 0.2) (layer "F.Cu") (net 5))
 (segment (start 158.115 104.86) (end 156.025 106.95) (width 0.2) (layer "F.Cu") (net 5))
 (segment (start 156.649999 89.4) (end 165.41 89.4) (width 0.2) (layer "F.Cu") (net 5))
 (segment (start 151.979999 84.73) (end 156.649999 89.4) (width 0.2) (layer "F.Cu") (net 5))
 (segment (start 146.17 82.720716) (end 148.179284 84.73) (width 0.2) (layer "F.Cu") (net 5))
 (segment (start 165.41 89.4) (end 165.41 93.11) (width 0.2) (layer "F.Cu") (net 5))
 (segment (start 163.19 93.13) (end 165.39 93.13) (width 0.2) (layer "F.Cu") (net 5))
 (segment (start 162.885 93.435) (end 163.19 93.13) (width 0.2) (layer "F.Cu") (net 5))
 (segment (start 165.39 93.13) (end 165.42 93.1) (width 0.2) (layer "F.Cu") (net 5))
 (segment (start 155.875 93.435) (end 162.885 93.435) (width 0.2) (layer "F.Cu") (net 5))
 (segment (start 155.3925 85.38) (end 163.06 85.38) (width 0.2) (layer "F.Cu") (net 9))
 (segment (start 163.06 85.38) (end 163.19 85.51) (width 0.2) (layer "F.Cu") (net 9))
 (segment (start 151.1675 82.3725) (end 151.17 82.37) (width 0.2) (layer "F.Cu") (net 6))
 (segment (start 155.875 94.705) (end 158.75 94.705) (width 0.2) (layer "F.Cu") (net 6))
 (segment (start 153.485 104.455) (end 153.47 104.44) (width 0.2) (layer "F.Cu") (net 6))
 (segment (start 162.225 94.705) (end 163.19 95.67) (width 0.2) (layer "F.Cu") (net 6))
 (segment (start 146.971788 79.884288) (end 151.1675 84.08) (width 0.2) (layer "F.Cu") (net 6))
 (segment (start 153.485 106.95) (end 153.485 104.455) (width 0.2) (layer "F.Cu") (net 6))
 (segment (start 146.17 79.884288) (end 146.971788 79.884288) (width 0.2) (layer "F.Cu") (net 6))
 (segment (start 158.75 94.705) (end 162.225 94.705) (width 0.2) (layer "F.Cu") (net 6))
 (segment (start 151.1675 84.08) (end 151.1675 82.3725) (width 0.2) (layer "F.Cu") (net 6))
 (via (at 151.17 82.37) (size 0.6) (drill 0.3) (layers "F.Cu" "B.Cu") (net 6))
 (via (at 153.47 104.44) (size 0.6) (drill 0.3) (layers "F.Cu" "B.Cu") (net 6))
 (via (at 158.75 94.705) (size 0.6) (drill 0.3) (layers "F.Cu" "B.Cu") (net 6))
 (segment (start 158.75 104.44) (end 153.47 104.44) (width 0.2) (layer "B.Cu") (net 6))
 (segment (start 158.75 94.705) (end 158.75 82.37) (width 0.2) (layer "B.Cu") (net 6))
 (segment (start 158.75 94.705) (end 158.75 104.44) (width 0.2) (layer "B.Cu") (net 6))
 (segment (start 158.75 82.37) (end 151.17 82.37) (width 0.2) (layer "B.Cu") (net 6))
 (segment (start 155.3925 86.03) (end 161.17 86.03) (width 0.2) (layer "F.Cu") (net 8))
 (segment (start 161.17 86.03) (end 163.19 88.05) (width 0.2) (layer "F.Cu") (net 8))
 (segment (start 150.965 93.435) (end 148.565 93.435) (width 0.2) (layer "F.Cu") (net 14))
 (segment (start 139.73 94.26) (end 132.15 94.26) (width 0.2) (layer "F.Cu") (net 14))
 (segment (start 148.565 93.435) (end 147.77 94.23) (width 0.2) (layer "F.Cu") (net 14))
 (segment (start 132.15 94.26) (end 130.01 92.12) (width 0.2) (layer "F.Cu") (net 14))
 (via (at 147.77 94.23) (size 0.6) (drill 0.3) (layers "F.Cu" "B.Cu") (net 14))
 (via (at 139.73 94.26) (size 0.6) (drill 0.3) (layers "F.Cu" "B.Cu") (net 14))
 (segment (start 147.77 94.23) (end 139.76 94.23) (width 0.2) (layer "B.Cu") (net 14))
 (segment (start 139.76 94.23) (end 139.73 94.26) (width 0.2) (layer "B.Cu") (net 14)))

